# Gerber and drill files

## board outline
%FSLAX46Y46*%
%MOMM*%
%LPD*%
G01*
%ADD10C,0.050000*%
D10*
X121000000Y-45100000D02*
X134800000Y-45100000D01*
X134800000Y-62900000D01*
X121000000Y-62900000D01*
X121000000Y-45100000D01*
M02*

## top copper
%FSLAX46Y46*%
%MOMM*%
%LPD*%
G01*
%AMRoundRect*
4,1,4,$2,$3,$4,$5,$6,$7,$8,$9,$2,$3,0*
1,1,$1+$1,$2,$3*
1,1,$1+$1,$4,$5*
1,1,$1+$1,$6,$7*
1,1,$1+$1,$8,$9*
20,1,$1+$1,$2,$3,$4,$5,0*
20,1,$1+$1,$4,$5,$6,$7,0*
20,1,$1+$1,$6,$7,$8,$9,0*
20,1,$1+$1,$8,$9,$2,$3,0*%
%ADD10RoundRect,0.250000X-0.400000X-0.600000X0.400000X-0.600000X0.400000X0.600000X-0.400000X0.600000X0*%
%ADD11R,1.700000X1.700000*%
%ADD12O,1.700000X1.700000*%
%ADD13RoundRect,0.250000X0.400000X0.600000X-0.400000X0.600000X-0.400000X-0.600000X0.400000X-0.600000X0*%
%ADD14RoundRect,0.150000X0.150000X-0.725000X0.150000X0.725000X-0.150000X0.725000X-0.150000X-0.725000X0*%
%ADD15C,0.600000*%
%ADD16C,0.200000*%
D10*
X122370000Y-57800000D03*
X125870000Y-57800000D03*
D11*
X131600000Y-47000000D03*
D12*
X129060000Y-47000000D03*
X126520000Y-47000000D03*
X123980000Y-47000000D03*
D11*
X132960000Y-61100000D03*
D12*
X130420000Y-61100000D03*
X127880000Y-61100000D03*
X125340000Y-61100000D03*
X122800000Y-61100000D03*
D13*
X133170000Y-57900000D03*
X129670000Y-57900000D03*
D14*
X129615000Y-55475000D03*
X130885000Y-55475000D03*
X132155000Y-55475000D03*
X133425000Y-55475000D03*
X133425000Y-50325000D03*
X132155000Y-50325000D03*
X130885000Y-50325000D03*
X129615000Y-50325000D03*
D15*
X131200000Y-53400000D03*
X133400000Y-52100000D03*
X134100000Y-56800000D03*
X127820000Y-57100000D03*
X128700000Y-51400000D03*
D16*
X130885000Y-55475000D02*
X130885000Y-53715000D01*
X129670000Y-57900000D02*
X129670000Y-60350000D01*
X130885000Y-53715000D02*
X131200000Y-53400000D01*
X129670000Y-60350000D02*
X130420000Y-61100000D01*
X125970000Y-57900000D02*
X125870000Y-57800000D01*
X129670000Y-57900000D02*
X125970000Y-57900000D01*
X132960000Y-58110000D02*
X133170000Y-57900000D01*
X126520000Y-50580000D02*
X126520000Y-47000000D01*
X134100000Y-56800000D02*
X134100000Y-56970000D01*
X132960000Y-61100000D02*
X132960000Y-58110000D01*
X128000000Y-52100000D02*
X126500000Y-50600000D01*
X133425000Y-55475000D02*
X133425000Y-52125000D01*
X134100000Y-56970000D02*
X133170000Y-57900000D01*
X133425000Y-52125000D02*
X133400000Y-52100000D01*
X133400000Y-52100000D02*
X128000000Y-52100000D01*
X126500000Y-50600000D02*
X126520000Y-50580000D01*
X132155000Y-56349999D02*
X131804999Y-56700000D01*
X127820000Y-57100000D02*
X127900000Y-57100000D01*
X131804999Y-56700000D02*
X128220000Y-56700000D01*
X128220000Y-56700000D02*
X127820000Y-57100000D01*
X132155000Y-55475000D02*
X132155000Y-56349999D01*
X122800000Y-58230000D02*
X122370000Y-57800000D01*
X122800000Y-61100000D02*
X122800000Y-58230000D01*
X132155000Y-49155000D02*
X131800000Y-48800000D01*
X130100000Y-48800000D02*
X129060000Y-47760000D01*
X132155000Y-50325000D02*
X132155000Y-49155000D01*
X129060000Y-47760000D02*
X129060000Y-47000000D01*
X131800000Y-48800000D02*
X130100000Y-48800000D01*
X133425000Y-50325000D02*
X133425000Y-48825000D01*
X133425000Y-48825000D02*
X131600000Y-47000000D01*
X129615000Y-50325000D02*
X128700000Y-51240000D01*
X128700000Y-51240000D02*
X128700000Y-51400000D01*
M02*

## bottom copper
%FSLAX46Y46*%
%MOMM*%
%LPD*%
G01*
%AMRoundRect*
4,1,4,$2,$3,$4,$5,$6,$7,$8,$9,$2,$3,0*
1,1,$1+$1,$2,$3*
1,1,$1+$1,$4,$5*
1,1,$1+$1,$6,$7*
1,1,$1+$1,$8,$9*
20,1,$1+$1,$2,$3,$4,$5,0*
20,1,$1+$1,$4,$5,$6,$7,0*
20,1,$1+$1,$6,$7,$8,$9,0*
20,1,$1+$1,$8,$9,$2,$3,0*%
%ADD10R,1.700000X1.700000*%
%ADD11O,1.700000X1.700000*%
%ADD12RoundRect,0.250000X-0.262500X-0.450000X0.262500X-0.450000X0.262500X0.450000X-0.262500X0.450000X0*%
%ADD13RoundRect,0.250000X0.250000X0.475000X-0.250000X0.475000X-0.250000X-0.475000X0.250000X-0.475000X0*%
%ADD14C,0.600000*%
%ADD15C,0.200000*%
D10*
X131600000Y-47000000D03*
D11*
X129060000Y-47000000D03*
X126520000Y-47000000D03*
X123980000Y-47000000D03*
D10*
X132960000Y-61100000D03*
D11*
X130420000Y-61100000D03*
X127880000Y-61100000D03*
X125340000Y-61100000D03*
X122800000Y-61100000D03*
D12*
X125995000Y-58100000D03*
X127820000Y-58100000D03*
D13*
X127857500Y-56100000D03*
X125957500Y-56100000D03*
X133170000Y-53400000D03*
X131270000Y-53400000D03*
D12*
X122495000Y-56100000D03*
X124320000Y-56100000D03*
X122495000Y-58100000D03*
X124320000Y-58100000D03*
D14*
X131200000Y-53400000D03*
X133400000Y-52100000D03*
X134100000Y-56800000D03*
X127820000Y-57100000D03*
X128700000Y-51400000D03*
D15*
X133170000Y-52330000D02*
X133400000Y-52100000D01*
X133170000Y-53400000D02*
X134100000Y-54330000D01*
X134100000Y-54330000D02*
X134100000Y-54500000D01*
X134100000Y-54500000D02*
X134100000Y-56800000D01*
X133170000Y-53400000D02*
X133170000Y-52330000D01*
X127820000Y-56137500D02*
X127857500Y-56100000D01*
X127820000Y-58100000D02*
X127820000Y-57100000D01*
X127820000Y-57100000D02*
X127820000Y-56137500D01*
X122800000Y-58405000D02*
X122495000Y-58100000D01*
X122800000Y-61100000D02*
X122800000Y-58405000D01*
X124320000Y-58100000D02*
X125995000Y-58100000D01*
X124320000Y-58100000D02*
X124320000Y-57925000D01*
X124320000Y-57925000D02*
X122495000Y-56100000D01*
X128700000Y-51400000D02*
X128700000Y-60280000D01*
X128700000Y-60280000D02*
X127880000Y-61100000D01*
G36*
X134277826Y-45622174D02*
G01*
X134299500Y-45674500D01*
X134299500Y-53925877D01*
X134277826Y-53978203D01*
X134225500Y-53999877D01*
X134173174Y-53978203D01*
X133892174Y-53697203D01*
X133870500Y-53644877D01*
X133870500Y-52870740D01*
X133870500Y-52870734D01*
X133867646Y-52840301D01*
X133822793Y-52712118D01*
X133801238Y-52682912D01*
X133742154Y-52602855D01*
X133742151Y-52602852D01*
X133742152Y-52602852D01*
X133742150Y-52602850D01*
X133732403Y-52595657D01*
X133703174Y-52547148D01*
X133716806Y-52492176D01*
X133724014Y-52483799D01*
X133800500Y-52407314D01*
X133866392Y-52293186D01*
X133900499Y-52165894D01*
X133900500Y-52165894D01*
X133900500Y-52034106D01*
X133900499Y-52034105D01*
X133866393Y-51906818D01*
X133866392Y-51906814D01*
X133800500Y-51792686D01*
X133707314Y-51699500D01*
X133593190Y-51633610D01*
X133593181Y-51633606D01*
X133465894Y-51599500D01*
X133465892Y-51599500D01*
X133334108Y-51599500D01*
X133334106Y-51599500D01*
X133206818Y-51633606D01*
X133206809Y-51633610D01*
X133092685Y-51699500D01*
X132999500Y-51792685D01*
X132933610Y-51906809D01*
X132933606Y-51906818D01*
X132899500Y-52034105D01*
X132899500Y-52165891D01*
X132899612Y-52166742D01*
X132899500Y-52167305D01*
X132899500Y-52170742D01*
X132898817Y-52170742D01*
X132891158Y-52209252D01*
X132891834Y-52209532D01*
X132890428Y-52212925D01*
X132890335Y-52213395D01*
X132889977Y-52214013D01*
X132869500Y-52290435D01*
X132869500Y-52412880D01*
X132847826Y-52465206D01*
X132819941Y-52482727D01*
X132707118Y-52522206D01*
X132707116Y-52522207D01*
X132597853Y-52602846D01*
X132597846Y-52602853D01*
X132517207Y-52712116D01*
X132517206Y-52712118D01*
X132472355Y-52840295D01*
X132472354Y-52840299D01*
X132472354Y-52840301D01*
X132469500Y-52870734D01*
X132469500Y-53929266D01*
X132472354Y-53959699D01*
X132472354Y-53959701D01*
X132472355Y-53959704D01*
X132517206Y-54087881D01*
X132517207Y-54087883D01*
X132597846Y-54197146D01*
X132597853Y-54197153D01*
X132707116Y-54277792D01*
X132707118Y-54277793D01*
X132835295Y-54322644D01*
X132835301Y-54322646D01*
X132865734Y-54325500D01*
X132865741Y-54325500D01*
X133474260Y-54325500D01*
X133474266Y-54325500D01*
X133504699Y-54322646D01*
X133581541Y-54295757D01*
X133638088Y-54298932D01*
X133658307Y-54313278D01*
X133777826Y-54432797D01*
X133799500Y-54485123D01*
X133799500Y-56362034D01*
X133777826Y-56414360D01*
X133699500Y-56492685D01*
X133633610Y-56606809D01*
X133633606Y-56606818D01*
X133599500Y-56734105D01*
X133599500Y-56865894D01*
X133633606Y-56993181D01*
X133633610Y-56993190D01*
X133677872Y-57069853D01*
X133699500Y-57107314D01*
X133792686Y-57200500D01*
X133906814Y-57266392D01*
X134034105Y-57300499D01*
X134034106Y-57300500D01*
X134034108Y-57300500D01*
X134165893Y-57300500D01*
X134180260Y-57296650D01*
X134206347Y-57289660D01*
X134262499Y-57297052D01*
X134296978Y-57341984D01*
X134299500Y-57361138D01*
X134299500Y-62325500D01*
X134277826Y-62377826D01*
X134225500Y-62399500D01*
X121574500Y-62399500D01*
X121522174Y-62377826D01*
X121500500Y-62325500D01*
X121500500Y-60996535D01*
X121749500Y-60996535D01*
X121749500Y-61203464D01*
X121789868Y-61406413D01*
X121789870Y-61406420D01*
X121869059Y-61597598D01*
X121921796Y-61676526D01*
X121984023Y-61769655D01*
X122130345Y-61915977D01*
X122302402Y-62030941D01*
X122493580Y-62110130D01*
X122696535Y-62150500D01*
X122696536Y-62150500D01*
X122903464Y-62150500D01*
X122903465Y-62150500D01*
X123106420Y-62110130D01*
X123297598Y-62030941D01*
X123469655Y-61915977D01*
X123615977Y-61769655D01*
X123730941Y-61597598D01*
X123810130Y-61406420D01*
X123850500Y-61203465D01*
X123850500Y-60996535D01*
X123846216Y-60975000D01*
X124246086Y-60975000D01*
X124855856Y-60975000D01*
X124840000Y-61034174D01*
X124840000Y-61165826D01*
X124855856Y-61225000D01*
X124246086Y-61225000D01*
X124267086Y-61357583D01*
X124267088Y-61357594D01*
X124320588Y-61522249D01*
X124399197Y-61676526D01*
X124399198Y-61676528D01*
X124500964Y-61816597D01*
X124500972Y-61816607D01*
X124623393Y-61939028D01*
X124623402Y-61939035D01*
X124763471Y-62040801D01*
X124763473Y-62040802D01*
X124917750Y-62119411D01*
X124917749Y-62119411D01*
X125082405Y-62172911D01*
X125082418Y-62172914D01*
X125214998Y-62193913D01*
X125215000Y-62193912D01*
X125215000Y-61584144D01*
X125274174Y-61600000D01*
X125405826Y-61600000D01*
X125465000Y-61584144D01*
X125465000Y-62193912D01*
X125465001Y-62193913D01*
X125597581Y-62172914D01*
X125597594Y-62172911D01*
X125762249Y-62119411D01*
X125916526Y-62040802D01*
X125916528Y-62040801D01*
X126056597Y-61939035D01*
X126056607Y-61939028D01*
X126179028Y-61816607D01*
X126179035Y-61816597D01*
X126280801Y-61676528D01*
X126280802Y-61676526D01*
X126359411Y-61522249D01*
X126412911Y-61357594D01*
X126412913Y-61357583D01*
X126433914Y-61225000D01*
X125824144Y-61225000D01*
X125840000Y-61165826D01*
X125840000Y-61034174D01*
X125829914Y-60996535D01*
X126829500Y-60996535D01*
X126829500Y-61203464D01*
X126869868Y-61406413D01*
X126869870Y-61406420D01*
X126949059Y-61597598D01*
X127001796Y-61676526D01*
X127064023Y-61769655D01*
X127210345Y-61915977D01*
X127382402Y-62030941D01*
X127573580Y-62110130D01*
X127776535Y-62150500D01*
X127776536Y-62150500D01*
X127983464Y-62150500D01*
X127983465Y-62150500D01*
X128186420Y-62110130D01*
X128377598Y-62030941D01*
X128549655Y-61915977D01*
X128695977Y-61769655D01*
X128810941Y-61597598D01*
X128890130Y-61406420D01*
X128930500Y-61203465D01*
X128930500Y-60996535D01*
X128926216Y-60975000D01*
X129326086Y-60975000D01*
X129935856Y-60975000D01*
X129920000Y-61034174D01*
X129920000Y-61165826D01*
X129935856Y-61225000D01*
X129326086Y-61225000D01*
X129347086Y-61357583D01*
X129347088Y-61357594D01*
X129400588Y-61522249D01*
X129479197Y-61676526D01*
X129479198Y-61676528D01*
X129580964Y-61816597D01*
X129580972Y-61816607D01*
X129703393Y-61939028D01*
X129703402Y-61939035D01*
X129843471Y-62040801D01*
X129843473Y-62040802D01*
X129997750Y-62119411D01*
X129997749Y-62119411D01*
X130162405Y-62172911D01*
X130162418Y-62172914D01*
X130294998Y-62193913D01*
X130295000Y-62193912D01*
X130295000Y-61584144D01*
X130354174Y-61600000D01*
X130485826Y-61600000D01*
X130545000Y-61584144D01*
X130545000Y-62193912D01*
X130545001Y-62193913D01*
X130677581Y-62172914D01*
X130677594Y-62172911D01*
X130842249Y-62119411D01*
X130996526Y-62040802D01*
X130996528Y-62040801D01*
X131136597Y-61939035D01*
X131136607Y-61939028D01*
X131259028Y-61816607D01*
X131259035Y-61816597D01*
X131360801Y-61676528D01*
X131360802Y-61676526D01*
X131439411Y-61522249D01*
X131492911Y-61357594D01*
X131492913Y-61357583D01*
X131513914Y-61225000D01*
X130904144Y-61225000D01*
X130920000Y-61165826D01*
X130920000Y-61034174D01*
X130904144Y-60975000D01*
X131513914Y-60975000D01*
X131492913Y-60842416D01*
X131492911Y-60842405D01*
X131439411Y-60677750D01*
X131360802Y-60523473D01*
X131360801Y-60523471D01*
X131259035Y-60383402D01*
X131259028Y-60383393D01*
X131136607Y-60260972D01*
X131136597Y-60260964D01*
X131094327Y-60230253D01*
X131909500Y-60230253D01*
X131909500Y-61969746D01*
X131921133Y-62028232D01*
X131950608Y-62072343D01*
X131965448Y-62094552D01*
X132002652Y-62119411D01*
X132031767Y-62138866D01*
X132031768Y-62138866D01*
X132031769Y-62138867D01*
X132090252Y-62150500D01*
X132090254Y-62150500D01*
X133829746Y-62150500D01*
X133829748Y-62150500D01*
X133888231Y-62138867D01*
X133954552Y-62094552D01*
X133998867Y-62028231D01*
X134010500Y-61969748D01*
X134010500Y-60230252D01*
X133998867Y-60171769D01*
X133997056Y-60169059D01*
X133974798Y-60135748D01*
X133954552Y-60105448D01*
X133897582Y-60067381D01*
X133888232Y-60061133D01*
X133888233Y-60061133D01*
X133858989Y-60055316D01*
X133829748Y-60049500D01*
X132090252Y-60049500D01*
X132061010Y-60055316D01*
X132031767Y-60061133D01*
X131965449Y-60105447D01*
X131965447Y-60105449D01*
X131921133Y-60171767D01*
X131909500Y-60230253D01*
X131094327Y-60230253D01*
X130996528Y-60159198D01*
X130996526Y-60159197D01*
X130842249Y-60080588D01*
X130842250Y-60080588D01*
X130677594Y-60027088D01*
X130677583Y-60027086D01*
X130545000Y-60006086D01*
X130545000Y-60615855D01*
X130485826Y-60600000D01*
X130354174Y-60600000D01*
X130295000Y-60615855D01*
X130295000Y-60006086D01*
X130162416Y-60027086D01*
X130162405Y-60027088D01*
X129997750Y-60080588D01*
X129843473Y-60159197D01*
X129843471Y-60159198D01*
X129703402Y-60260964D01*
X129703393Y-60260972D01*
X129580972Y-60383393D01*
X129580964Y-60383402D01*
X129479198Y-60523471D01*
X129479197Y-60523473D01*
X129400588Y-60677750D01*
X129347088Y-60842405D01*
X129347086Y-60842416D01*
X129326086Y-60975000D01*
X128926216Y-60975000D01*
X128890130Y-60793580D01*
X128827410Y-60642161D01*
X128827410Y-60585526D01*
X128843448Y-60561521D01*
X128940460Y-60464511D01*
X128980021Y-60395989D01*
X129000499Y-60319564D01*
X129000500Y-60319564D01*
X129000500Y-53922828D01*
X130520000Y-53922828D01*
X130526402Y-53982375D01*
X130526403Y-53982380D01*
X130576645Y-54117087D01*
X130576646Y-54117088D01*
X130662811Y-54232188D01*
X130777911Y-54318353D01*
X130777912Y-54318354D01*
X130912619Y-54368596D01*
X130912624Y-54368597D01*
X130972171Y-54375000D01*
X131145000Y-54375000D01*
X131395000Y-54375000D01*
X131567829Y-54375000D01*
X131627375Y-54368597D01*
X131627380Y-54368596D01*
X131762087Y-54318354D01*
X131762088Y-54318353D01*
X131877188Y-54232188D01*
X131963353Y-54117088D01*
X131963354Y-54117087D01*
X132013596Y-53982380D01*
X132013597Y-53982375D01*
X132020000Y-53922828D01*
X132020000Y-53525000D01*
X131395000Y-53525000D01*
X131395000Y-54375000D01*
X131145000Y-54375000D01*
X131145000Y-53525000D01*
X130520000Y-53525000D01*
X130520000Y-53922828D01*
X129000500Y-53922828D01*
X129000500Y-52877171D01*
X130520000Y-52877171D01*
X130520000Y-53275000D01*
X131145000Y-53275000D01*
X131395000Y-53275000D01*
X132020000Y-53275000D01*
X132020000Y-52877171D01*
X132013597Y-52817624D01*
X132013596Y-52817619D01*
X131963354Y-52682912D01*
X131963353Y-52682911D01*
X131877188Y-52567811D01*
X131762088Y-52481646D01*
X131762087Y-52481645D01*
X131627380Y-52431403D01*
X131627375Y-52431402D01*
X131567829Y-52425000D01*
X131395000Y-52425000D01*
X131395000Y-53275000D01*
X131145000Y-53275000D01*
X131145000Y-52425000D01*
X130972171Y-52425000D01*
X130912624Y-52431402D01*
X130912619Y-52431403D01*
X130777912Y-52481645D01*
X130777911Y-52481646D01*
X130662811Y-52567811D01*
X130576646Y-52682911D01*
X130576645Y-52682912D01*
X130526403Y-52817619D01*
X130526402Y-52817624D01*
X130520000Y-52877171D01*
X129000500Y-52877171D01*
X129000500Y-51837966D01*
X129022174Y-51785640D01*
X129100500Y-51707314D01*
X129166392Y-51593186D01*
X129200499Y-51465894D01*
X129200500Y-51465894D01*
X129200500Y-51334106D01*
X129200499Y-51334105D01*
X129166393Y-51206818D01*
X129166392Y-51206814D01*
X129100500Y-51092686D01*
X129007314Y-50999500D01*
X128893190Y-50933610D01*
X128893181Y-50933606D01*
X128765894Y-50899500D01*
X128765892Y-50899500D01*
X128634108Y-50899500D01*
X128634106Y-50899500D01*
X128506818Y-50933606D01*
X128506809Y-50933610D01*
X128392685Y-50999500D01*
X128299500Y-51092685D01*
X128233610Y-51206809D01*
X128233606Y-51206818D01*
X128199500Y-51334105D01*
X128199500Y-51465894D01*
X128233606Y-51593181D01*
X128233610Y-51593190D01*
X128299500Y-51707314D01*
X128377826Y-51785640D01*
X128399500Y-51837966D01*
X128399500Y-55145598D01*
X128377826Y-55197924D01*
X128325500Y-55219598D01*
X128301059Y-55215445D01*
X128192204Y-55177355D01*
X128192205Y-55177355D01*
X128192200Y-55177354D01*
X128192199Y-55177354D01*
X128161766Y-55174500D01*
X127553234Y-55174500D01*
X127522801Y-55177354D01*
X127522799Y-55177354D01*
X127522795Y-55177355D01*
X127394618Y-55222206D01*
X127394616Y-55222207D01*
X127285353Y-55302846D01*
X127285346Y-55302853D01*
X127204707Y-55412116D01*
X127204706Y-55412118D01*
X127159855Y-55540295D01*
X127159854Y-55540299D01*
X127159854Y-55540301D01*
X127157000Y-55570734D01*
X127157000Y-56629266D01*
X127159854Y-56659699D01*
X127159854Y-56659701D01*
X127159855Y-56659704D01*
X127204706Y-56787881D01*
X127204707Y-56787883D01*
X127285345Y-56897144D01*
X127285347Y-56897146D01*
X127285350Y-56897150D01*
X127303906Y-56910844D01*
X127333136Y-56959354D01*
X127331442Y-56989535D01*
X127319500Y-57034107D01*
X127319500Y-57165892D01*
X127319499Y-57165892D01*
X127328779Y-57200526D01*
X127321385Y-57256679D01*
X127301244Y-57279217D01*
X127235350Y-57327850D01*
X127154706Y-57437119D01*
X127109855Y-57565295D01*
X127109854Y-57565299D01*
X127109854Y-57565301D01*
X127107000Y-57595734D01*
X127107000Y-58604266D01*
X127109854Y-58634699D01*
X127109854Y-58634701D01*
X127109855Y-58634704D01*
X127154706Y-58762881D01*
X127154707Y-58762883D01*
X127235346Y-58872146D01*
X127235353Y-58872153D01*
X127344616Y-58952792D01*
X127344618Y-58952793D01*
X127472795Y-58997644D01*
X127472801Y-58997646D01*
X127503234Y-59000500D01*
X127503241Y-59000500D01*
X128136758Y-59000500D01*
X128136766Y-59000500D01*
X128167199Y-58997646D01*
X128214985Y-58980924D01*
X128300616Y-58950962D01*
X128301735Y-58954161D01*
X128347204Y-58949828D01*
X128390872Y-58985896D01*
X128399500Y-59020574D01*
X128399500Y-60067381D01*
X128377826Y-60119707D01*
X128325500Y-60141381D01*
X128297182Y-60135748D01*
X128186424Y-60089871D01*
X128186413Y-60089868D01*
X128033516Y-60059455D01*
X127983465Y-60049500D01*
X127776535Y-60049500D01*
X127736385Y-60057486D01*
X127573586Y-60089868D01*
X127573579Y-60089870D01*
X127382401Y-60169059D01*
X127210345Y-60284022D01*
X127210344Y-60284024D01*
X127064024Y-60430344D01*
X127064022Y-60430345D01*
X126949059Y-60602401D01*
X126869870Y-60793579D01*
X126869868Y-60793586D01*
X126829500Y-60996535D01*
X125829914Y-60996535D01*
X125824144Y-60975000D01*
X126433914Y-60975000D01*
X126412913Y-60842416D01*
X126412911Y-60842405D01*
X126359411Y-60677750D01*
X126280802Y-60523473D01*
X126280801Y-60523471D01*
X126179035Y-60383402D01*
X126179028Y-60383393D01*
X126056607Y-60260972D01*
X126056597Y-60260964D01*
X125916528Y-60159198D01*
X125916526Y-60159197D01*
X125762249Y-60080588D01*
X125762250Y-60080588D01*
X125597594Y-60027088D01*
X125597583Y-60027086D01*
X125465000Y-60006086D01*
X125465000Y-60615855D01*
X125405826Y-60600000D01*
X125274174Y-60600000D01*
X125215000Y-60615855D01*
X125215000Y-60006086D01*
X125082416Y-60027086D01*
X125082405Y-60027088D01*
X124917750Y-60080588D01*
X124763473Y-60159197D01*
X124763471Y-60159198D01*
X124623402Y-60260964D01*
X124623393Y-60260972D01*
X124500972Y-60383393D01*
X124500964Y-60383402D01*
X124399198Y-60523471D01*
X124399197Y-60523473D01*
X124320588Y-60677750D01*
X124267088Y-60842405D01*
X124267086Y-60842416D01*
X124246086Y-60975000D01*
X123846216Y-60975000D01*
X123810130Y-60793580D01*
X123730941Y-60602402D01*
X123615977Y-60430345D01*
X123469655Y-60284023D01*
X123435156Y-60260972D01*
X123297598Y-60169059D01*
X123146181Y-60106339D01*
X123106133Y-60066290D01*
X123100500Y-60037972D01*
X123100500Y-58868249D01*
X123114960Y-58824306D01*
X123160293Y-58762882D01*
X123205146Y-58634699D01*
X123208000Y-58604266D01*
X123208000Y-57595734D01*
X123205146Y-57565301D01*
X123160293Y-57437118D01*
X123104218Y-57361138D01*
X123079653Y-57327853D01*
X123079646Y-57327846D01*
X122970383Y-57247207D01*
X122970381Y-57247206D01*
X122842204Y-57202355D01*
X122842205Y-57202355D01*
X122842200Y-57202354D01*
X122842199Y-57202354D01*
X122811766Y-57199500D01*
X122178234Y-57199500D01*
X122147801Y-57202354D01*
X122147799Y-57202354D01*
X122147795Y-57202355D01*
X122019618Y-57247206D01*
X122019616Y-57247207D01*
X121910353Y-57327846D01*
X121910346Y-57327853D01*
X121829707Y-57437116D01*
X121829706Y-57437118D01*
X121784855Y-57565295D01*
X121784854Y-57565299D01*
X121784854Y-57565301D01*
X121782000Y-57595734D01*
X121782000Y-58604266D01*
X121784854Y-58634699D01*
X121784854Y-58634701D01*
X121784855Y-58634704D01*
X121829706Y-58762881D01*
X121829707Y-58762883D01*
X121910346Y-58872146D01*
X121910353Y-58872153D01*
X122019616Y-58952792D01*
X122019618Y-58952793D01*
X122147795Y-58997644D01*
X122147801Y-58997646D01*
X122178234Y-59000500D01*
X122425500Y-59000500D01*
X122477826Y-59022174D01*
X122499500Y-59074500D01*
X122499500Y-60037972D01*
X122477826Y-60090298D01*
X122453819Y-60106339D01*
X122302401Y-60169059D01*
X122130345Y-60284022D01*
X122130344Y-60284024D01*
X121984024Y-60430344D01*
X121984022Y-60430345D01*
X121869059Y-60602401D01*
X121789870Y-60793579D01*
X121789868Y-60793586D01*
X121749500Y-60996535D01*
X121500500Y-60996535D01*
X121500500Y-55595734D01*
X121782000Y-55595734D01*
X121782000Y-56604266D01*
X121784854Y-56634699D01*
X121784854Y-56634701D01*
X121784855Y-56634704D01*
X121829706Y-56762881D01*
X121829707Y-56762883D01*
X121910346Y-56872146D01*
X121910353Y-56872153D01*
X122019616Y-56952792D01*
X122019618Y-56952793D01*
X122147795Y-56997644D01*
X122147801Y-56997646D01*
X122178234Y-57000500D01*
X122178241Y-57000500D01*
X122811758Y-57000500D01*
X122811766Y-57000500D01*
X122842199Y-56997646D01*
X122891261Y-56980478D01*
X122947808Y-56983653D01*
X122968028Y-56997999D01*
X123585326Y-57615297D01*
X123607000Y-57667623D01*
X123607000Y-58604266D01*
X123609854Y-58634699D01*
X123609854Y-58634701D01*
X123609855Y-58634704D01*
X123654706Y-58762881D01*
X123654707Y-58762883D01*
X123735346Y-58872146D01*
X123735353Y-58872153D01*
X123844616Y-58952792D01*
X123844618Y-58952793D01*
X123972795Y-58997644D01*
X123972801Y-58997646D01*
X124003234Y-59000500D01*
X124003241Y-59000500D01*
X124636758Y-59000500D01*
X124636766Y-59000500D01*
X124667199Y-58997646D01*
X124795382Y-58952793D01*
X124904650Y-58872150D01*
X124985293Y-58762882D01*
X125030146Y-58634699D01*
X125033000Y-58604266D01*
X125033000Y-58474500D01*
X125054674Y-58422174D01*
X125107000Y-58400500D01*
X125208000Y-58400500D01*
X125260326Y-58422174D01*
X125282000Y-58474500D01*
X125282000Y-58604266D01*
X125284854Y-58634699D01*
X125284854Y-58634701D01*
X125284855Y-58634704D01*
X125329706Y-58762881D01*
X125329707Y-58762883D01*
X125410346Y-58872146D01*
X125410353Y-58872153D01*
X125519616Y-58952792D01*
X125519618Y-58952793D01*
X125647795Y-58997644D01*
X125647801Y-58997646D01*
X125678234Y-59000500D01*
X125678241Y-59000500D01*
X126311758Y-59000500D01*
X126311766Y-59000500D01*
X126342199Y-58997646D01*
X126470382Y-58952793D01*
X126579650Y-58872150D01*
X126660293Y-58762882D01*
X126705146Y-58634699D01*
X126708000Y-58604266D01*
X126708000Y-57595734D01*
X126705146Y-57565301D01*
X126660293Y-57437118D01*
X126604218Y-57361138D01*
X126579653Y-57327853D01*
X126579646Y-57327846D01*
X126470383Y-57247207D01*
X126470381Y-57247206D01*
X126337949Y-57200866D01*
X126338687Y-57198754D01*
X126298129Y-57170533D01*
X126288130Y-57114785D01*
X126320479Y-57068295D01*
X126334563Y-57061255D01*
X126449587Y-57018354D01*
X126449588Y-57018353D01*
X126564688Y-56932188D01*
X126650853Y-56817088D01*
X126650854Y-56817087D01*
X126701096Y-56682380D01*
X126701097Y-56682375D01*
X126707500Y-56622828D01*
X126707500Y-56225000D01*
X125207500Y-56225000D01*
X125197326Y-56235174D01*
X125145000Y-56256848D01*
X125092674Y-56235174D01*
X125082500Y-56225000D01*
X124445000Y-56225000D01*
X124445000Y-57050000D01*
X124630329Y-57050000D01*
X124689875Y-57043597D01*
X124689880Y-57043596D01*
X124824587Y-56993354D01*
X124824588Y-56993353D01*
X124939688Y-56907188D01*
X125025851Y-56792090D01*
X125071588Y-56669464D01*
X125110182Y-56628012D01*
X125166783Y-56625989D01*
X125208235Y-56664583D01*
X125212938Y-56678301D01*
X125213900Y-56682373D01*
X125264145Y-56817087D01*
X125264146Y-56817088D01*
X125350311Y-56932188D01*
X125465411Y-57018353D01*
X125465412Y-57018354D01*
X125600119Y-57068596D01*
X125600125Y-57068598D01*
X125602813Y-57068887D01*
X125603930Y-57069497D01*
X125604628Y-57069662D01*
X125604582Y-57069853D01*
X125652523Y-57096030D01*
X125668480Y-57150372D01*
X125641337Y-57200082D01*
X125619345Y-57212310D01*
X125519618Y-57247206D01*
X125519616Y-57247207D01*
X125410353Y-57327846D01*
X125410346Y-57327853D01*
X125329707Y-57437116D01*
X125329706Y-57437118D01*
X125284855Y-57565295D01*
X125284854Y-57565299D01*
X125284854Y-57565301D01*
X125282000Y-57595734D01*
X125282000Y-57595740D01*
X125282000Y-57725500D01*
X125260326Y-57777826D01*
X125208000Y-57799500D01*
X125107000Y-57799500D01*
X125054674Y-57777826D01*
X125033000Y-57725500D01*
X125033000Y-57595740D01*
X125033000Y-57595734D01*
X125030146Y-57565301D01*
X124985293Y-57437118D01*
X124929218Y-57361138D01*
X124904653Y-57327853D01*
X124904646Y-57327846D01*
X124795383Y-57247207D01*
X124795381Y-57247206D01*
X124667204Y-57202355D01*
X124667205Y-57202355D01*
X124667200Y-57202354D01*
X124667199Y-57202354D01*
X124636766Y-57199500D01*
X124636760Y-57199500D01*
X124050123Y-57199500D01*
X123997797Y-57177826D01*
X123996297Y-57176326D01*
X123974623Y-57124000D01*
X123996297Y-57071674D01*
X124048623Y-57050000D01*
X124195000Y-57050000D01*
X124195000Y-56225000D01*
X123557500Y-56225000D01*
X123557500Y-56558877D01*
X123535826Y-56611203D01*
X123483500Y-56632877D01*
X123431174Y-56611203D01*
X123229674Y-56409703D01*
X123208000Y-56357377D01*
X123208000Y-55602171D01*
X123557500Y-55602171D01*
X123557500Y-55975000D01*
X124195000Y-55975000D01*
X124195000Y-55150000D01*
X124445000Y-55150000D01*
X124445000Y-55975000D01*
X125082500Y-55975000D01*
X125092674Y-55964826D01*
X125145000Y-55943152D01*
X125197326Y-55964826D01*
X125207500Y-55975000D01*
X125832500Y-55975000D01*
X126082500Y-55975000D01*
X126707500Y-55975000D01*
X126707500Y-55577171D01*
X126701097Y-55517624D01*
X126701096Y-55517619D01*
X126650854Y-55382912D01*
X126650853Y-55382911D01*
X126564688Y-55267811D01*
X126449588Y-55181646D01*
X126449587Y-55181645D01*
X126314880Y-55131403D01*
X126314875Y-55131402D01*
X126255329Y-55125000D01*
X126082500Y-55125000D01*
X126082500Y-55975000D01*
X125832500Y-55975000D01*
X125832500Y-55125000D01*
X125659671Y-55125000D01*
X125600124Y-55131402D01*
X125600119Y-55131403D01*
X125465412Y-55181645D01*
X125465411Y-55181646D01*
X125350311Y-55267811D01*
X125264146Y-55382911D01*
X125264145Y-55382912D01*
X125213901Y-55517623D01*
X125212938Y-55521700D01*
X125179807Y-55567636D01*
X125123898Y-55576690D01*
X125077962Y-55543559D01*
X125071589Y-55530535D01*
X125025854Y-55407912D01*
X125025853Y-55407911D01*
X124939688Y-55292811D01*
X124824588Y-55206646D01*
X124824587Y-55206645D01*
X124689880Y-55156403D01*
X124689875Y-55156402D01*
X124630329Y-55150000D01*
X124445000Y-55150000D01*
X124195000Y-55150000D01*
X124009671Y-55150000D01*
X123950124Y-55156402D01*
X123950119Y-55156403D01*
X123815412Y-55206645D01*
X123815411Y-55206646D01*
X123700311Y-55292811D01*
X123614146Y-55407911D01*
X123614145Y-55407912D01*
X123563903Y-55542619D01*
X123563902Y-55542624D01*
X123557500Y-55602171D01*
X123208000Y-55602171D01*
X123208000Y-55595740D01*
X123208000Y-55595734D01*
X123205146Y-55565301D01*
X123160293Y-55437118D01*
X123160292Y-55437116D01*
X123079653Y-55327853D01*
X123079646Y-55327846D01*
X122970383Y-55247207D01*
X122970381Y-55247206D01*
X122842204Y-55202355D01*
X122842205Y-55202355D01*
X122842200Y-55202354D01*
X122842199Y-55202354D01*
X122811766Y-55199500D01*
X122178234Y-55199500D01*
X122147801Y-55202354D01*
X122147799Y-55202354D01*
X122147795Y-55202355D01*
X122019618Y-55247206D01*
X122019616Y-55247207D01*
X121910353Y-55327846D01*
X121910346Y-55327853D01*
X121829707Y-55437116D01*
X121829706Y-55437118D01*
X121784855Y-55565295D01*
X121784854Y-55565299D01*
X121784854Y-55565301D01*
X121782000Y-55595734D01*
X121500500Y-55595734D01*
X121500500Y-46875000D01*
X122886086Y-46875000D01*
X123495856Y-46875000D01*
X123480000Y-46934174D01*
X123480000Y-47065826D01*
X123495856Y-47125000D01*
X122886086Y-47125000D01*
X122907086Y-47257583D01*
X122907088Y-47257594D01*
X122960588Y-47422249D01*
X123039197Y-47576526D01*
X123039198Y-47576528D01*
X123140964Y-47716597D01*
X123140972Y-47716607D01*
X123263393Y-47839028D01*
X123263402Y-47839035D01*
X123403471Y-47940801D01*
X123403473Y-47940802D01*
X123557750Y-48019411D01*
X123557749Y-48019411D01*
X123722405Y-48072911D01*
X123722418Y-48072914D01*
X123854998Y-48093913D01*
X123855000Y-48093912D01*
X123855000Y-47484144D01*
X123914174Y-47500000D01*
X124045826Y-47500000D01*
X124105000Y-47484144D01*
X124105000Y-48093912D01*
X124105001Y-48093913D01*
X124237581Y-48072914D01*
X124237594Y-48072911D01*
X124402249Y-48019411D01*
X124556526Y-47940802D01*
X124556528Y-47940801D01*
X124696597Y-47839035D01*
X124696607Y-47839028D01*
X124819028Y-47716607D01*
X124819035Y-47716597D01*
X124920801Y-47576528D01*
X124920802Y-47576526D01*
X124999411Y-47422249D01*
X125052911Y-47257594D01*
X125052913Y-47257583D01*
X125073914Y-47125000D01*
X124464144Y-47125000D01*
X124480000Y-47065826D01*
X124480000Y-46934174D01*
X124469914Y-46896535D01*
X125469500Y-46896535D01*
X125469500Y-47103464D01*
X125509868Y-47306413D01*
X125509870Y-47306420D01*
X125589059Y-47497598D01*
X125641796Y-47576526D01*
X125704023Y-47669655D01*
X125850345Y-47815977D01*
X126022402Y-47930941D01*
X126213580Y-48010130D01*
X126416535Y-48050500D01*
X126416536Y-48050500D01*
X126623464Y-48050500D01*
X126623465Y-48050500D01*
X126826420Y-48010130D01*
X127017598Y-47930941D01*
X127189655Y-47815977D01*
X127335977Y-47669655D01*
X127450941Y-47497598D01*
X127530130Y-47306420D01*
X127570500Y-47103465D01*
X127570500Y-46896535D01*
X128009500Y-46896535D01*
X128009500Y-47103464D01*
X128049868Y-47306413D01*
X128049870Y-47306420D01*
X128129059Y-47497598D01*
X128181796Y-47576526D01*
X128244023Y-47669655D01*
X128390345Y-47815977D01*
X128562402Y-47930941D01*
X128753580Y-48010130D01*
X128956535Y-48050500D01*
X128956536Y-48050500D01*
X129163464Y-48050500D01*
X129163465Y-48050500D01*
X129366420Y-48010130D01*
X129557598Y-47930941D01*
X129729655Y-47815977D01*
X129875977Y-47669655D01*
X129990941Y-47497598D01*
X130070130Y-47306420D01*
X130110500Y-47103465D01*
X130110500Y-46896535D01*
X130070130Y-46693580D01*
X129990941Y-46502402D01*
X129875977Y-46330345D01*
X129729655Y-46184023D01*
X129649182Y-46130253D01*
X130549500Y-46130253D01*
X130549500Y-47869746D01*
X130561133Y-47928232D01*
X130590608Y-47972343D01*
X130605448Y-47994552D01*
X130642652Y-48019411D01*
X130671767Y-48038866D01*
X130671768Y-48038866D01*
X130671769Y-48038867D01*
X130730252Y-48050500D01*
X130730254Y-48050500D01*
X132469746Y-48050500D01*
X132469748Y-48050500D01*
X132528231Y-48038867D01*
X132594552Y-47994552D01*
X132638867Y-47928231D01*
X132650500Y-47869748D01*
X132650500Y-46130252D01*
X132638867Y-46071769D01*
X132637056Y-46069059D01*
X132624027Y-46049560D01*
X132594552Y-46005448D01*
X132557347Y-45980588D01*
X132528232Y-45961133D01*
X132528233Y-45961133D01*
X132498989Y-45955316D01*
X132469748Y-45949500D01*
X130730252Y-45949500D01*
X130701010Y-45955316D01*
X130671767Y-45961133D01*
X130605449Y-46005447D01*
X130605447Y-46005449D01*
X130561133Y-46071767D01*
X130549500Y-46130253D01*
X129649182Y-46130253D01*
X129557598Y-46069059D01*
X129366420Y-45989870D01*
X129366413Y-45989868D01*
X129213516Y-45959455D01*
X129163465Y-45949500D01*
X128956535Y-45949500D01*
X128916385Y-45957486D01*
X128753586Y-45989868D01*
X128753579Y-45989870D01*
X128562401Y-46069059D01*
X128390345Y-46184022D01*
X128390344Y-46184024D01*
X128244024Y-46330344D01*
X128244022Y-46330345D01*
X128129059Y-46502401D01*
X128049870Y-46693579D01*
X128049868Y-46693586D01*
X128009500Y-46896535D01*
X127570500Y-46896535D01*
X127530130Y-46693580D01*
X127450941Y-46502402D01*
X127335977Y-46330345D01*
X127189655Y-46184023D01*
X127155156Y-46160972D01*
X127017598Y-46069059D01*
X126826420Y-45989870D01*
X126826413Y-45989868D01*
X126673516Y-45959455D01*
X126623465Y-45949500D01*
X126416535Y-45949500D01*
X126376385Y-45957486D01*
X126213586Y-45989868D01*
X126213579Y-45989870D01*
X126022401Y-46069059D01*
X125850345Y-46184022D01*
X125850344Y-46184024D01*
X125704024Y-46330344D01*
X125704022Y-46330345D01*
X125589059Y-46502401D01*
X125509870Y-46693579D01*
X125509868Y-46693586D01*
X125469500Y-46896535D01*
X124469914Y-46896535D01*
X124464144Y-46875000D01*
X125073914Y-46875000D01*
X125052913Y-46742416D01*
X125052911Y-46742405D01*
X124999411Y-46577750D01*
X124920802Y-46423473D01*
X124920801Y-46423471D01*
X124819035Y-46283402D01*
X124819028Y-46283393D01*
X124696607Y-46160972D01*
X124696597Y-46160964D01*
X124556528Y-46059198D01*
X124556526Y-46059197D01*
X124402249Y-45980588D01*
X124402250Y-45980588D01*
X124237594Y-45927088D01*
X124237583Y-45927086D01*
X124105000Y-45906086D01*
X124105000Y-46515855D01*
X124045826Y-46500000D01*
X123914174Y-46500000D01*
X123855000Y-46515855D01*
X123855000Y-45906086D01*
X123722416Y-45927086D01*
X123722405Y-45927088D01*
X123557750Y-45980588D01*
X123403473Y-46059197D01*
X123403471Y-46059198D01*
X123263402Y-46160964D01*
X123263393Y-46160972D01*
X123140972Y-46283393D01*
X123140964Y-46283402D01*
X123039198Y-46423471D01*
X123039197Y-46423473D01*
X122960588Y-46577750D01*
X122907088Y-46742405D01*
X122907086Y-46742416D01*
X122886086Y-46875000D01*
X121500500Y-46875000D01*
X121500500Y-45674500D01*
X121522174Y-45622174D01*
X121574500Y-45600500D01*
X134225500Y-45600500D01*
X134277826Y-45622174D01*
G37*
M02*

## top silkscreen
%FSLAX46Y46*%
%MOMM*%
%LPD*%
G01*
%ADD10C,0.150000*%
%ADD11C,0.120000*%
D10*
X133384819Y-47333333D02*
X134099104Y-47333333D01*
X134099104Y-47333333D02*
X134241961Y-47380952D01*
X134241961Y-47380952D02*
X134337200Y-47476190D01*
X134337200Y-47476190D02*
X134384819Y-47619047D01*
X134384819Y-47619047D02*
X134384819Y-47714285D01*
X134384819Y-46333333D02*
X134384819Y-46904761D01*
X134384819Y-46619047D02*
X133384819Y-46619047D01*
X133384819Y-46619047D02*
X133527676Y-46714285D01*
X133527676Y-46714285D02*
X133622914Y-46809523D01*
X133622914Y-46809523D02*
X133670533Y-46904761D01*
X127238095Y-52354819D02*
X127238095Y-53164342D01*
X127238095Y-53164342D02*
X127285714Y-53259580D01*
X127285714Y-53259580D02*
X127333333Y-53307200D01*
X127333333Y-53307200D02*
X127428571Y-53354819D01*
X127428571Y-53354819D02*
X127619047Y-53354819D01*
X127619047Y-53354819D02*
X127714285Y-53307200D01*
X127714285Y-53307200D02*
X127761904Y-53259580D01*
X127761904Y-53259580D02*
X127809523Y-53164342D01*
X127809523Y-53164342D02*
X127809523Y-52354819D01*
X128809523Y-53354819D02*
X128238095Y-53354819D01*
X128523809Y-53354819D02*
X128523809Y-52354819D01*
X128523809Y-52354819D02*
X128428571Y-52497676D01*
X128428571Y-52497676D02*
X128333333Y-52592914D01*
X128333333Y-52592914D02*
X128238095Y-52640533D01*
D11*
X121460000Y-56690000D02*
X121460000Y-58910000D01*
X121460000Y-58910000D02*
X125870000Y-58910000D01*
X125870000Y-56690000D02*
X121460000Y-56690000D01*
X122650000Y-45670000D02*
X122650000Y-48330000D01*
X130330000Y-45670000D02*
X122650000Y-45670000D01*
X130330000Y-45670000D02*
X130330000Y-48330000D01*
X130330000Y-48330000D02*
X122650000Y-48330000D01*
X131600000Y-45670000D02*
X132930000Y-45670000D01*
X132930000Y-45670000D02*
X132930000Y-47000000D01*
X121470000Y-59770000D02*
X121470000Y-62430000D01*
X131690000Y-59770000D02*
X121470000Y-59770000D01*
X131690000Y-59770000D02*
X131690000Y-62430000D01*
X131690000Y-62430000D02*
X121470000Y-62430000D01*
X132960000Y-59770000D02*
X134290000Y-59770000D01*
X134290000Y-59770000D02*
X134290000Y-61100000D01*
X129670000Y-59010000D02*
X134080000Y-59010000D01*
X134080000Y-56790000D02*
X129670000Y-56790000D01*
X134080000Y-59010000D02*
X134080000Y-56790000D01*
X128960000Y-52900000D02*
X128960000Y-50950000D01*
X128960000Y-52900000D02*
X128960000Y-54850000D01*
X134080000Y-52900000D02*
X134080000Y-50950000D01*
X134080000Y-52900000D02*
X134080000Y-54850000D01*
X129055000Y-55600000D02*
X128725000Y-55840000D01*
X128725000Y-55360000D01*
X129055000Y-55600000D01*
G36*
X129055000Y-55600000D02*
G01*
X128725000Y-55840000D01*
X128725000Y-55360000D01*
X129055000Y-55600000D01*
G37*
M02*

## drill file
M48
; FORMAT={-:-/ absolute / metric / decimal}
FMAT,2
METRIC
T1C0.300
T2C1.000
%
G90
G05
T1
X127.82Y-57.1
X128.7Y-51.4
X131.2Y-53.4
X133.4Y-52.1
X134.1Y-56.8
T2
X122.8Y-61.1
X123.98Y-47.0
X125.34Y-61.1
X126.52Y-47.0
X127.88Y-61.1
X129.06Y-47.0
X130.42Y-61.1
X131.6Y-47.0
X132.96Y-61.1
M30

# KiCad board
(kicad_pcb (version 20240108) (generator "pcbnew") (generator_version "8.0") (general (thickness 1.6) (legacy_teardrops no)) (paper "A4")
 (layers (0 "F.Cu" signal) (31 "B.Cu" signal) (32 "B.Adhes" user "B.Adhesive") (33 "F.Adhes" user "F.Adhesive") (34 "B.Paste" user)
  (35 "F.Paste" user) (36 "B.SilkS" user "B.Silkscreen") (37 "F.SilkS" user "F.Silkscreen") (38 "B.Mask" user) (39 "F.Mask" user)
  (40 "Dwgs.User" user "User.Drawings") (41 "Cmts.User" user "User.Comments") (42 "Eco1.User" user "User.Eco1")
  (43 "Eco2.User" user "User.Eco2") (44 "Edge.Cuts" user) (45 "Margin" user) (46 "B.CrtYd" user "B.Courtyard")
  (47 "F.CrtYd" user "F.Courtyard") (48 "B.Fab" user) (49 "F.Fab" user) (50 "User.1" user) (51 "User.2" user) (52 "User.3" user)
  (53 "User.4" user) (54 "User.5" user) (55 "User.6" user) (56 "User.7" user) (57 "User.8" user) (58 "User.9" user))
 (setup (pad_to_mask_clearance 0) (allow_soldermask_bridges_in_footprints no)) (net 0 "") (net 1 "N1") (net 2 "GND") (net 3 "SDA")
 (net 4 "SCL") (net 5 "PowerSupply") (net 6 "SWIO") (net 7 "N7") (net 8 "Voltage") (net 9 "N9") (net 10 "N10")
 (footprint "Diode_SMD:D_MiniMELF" (layer "F.Cu") (at 124.12 57.8)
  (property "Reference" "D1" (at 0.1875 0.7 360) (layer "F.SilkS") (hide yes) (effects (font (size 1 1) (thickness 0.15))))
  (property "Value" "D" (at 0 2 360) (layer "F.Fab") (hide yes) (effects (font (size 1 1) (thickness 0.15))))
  (fp_line (start -2.66 -1.11) (end -2.66 1.11) (stroke (width 0.12) (type solid)) (layer "F.SilkS"))
  (fp_line (start -2.66 1.11) (end 1.75 1.11) (stroke (width 0.12) (type solid)) (layer "F.SilkS"))
  (fp_line (start 1.75 -1.11) (end -2.66 -1.11) (stroke (width 0.12) (type solid)) (layer "F.SilkS"))
  (pad "1" smd roundrect (at -1.75 0) (size 1.3 1.7) (layers "F.Cu" "F.Paste" "F.Mask") (roundrect_rratio 0.1923076923) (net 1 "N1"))
  (pad "2" smd roundrect (at 1.75 0) (size 1.3 1.7) (layers "F.Cu" "F.Paste" "F.Mask") (roundrect_rratio 0.1923076923) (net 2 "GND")))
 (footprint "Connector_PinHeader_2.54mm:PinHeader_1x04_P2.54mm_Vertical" (layer "F.Cu") (at 131.6 47 -90)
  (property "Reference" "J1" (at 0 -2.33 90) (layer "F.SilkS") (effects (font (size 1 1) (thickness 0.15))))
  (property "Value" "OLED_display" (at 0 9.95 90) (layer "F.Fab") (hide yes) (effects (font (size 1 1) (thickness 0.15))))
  (fp_line (start -1.33 8.95) (end 1.33 8.95) (stroke (width 0.12) (type solid)) (layer "F.SilkS"))
  (fp_line (start -1.33 1.27) (end -1.33 8.95) (stroke (width 0.12) (type solid)) (layer "F.SilkS"))
  (fp_line (start -1.33 1.27) (end 1.33 1.27) (stroke (width 0.12) (type solid)) (layer "F.SilkS"))
  (fp_line (start 1.33 1.27) (end 1.33 8.95) (stroke (width 0.12) (type solid)) (layer "F.SilkS"))
  (fp_line (start -1.33 0) (end -1.33 -1.33) (stroke (width 0.12) (type solid)) (layer "F.SilkS"))
  (fp_line (start -1.33 -1.33) (end 0 -1.33) (stroke (width 0.12) (type solid)) (layer "F.SilkS"))
  (pad "1" thru_hole rect (at 0 0 270) (size 1.7 1.7) (drill 1) (layers "*.Cu" "*.Mask") (remove_unused_layers no) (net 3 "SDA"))
  (pad "2" thru_hole oval (at 0 2.54 270) (size 1.7 1.7) (drill 1) (layers "*.Cu" "*.Mask") (remove_unused_layers no) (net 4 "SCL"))
  (pad "3" thru_hole oval (at 0 5.08 270) (size 1.7 1.7) (drill 1) (layers "*.Cu" "*.Mask") (remove_unused_layers no) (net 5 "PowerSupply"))
  (pad "4" thru_hole oval (at 0 7.62 270) (size 1.7 1.7) (drill 1) (layers "*.Cu" "*.Mask") (remove_unused_layers no) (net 2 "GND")))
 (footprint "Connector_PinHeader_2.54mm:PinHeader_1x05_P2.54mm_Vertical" (layer "F.Cu") (at 132.96 61.1 -90)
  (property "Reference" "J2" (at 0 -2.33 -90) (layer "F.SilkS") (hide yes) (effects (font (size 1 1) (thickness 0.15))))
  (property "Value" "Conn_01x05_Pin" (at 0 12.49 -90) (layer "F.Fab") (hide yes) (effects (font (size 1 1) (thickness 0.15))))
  (fp_line (start -1.33 11.49) (end 1.33 11.49) (stroke (width 0.12) (type solid)) (layer "F.SilkS"))
  (fp_line (start -1.33 1.27) (end -1.33 11.49) (stroke (width 0.12) (type solid)) (layer "F.SilkS"))
  (fp_line (start -1.33 1.27) (end 1.33 1.27) (stroke (width 0.12) (type solid)) (layer "F.SilkS"))
  (fp_line (start 1.33 1.27) (end 1.33 11.49) (stroke (width 0.12) (type solid)) (layer "F.SilkS"))
  (fp_line (start -1.33 0) (end -1.33 -1.33) (stroke (width 0.12) (type solid)) (layer "F.SilkS"))
  (fp_line (start -1.33 -1.33) (end 0 -1.33) (stroke (width 0.12) (type solid)) (layer "F.SilkS"))
  (pad "1" thru_hole rect (at 0 0 270) (size 1.7 1.7) (drill 1) (layers "*.Cu" "*.Mask") (remove_unused_layers no) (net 5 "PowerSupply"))
  (pad "2" thru_hole oval (at 0 2.54 270) (size 1.7 1.7) (drill 1) (layers "*.Cu" "*.Mask") (remove_unused_layers no) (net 2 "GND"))
  (pad "3" thru_hole oval (at 0 5.08 270) (size 1.7 1.7) (drill 1) (layers "*.Cu" "*.Mask") (remove_unused_layers no) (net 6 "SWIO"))
  (pad "4" thru_hole oval (at 0 7.62 270) (size 1.7 1.7) (drill 1) (layers "*.Cu" "*.Mask") (remove_unused_layers no) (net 2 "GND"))
  (pad "5" thru_hole oval (at 0 10.16 270) (size 1.7 1.7) (drill 1) (layers "*.Cu" "*.Mask") (remove_unused_layers no) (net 1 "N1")))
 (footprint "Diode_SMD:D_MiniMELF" (layer "F.Cu") (at 131.42 57.9 180)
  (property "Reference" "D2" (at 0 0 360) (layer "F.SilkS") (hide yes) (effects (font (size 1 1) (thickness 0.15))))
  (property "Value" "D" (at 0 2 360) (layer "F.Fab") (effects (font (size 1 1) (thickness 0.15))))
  (fp_line (start 1.75 -1.11) (end -2.66 -1.11) (stroke (width 0.12) (type solid)) (layer "F.SilkS"))
  (fp_line (start -2.66 1.11) (end 1.75 1.11) (stroke (width 0.12) (type solid)) (layer "F.SilkS"))
  (fp_line (start -2.66 -1.11) (end -2.66 1.11) (stroke (width 0.12) (type solid)) (layer "F.SilkS"))
  (pad "1" smd roundrect (at -1.75 0 180) (size 1.3 1.7) (layers "F.Cu" "F.Paste" "F.Mask") (roundrect_rratio 0.1923076923)
   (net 5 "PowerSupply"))
  (pad "2" smd roundrect (at 1.75 0 180) (size 1.3 1.7) (layers "F.Cu" "F.Paste" "F.Mask") (roundrect_rratio 0.1923076923) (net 2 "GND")))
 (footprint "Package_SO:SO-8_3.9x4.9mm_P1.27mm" (layer "F.Cu") (at 131.52 52.9 90)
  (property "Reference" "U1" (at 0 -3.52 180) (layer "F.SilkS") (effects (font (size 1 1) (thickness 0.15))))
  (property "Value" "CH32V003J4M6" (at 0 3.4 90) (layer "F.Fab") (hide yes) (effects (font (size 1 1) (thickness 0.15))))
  (fp_line (start 0 -2.56) (end 1.95 -2.56) (stroke (width 0.12) (type solid)) (layer "F.SilkS"))
  (fp_line (start 0 -2.56) (end -1.95 -2.56) (stroke (width 0.12) (type solid)) (layer "F.SilkS"))
  (fp_line (start 0 2.56) (end 1.95 2.56) (stroke (width 0.12) (type solid)) (layer "F.SilkS"))
  (fp_line (start 0 2.56) (end -1.95 2.56) (stroke (width 0.12) (type solid)) (layer "F.SilkS"))
  (fp_poly
   (pts (xy -2.7 -2.465) (xy -2.94 -2.795) (xy -2.46 -2.795) (xy -2.7 -2.465)) (stroke (width 0.12) (type solid)) (fill solid)
   (layer "F.SilkS"))
  (pad "1" smd roundrect (at -2.575 -1.905 90) (size 1.75 0.6) (layers "F.Cu" "F.Paste" "F.Mask") (roundrect_rratio 0.25) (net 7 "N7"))
  (pad "2" smd roundrect (at -2.575 -0.635 90) (size 1.75 0.6) (layers "F.Cu" "F.Paste" "F.Mask") (roundrect_rratio 0.25) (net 2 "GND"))
  (pad "3" smd roundrect (at -2.575 0.635 90) (size 1.75 0.6) (layers "F.Cu" "F.Paste" "F.Mask") (roundrect_rratio 0.25) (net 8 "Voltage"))
  (pad "4" smd roundrect (at -2.575 1.905 90) (size 1.75 0.6) (layers "F.Cu" "F.Paste" "F.Mask") (roundrect_rratio 0.25)
   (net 5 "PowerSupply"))
  (pad "5" smd roundrect (at 2.575 1.905 90) (size 1.75 0.6) (layers "F.Cu" "F.Paste" "F.Mask") (roundrect_rratio 0.25) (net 3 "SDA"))
  (pad "6" smd roundrect (at 2.575 0.635 90) (size 1.75 0.6) (layers "F.Cu" "F.Paste" "F.Mask") (roundrect_rratio 0.25) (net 4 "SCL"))
  (pad "7" smd roundrect (at 2.575 -0.635 90) (size 1.75 0.6) (layers "F.Cu" "F.Paste" "F.Mask") (roundrect_rratio 0.25) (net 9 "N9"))
  (pad "8" smd roundrect (at 2.575 -1.905 90) (size 1.75 0.6) (layers "F.Cu" "F.Paste" "F.Mask") (roundrect_rratio 0.25) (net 6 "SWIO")))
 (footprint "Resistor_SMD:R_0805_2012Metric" (layer "B.Cu") (at 126.9075 58.1)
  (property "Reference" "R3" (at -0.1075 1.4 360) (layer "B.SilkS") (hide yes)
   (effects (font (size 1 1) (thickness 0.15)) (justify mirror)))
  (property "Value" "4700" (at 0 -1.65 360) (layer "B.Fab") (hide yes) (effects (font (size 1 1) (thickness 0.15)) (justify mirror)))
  (pad "1" smd roundrect (at -0.9125 0) (size 1.025 1.4) (layers "B.Cu" "B.Paste" "B.Mask") (roundrect_rratio 0.243902) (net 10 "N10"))
  (pad "2" smd roundrect (at 0.9125 0) (size 1.025 1.4) (layers "B.Cu" "B.Paste" "B.Mask") (roundrect_rratio 0.243902) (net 8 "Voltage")))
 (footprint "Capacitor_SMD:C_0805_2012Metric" (layer "B.Cu") (at 126.9075 56.1 180)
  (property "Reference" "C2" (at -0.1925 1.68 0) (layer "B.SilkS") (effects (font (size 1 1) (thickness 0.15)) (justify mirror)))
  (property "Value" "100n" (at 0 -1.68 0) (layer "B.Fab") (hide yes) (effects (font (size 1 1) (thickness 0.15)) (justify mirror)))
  (pad "1" smd roundrect (at -0.95 0 180) (size 1 1.45) (layers "B.Cu" "B.Paste" "B.Mask") (roundrect_rratio 0.25) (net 8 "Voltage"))
  (pad "2" smd roundrect (at 0.95 0 180) (size 1 1.45) (layers "B.Cu" "B.Paste" "B.Mask") (roundrect_rratio 0.25) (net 2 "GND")))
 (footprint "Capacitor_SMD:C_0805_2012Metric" (layer "B.Cu") (at 132.22 53.4 180)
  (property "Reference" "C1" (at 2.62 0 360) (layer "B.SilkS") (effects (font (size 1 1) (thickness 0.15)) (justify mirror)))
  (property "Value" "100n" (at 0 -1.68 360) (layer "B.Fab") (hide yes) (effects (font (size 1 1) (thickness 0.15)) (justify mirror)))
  (pad "1" smd roundrect (at -0.95 0 180) (size 1 1.45) (layers "B.Cu" "B.Paste" "B.Mask") (roundrect_rratio 0.25) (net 5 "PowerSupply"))
  (pad "2" smd roundrect (at 0.95 0 180) (size 1 1.45) (layers "B.Cu" "B.Paste" "B.Mask") (roundrect_rratio 0.25) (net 2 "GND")))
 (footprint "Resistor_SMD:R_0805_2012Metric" (layer "B.Cu") (at 123.4075 56.1)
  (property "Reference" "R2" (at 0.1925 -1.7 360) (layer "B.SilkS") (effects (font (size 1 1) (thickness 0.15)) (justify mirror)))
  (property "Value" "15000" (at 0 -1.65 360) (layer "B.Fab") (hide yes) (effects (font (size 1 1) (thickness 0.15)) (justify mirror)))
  (pad "1" smd roundrect (at -0.9125 0) (size 1.025 1.4) (layers "B.Cu" "B.Paste" "B.Mask") (roundrect_rratio 0.243902) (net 10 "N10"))
  (pad "2" smd roundrect (at 0.9125 0) (size 1.025 1.4) (layers "B.Cu" "B.Paste" "B.Mask") (roundrect_rratio 0.243902) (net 2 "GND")))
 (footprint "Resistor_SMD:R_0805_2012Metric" (layer "B.Cu") (at 123.4075 58.1)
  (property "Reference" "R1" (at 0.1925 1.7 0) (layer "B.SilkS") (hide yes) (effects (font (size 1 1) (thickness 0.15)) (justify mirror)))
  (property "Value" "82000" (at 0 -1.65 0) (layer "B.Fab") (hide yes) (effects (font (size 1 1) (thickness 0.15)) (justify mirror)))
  (pad "1" smd roundrect (at -0.9125 0) (size 1.025 1.4) (layers "B.Cu" "B.Paste" "B.Mask") (roundrect_rratio 0.243902) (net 1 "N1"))
  (pad "2" smd roundrect (at 0.9125 0) (size 1.025 1.4) (layers "B.Cu" "B.Paste" "B.Mask") (roundrect_rratio 0.243902) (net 10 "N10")))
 (gr_rect (start 121 45.1) (end 134.8 62.9) (stroke (width 0.05) (type default)) (fill none) (layer "Edge.Cuts"))
 (segment (start 130.885 55.475) (end 130.885 53.715) (width 0.2) (layer "F.Cu") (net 2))
 (segment (start 129.67 57.9) (end 129.67 60.35) (width 0.2) (layer "F.Cu") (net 2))
 (segment (start 130.885 53.715) (end 131.2 53.4) (width 0.2) (layer "F.Cu") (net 2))
 (segment (start 129.67 60.35) (end 130.42 61.1) (width 0.2) (layer "F.Cu") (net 2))
 (segment (start 125.97 57.9) (end 125.87 57.8) (width 0.2) (layer "F.Cu") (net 2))
 (segment (start 129.67 57.9) (end 125.97 57.9) (width 0.2) (layer "F.Cu") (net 2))
 (via (at 131.2 53.4) (size 0.6) (drill 0.3) (layers "F.Cu" "B.Cu") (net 2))
 (segment (start 132.96 58.11) (end 133.17 57.9) (width 0.2) (layer "F.Cu") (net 5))
 (segment (start 126.52 50.58) (end 126.52 47) (width 0.2) (layer "F.Cu") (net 5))
 (segment (start 134.1 56.8) (end 134.1 56.97) (width 0.2) (layer "F.Cu") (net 5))
 (segment (start 132.96 61.1) (end 132.96 58.11) (width 0.2) (layer "F.Cu") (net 5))
 (segment (start 128 52.1) (end 126.5 50.6) (width 0.2) (layer "F.Cu") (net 5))
 (segment (start 133.425 55.475) (end 133.425 52.125) (width 0.2) (layer "F.Cu") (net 5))
 (segment (start 134.1 56.97) (end 133.17 57.9) (width 0.2) (layer "F.Cu") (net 5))
 (segment (start 133.425 52.125) (end 133.4 52.1) (width 0.2) (layer "F.Cu") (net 5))
 (segment (start 133.4 52.1) (end 128 52.1) (width 0.2) (layer "F.Cu") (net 5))
 (segment (start 126.5 50.6) (end 126.52 50.58) (width 0.2) (layer "F.Cu") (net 5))
 (via (at 133.4 52.1) (size 0.6) (drill 0.3) (layers "F.Cu" "B.Cu") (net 5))
 (via (at 134.1 56.8) (size 0.6) (drill 0.3) (layers "F.Cu" "B.Cu") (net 5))
 (segment (start 133.17 52.33) (end 133.4 52.1) (width 0.2) (layer "B.Cu") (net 5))
 (segment (start 133.17 53.4) (end 134.1 54.33) (width 0.2) (layer "B.Cu") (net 5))
 (segment (start 134.1 54.33) (end 134.1 54.5) (width 0.2) (layer "B.Cu") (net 5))
 (segment (start 134.1 54.5) (end 134.1 56.8) (width 0.2) (layer "B.Cu") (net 5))
 (segment (start 133.17 53.4) (end 133.17 52.33) (width 0.2) (layer "B.Cu") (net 5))
 (segment (start 132.155 56.349999) (end 131.804999 56.7) (width 0.2) (layer "F.Cu") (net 8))
 (segment (start 127.82 57.1) (end 127.9 57.1) (width 0.2) (layer "F.Cu") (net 8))
 (segment (start 131.804999 56.7) (end 128.22 56.7) (width 0.2) (layer "F.Cu") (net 8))
 (segment (start 128.22 56.7) (end 127.82 57.1) (width 0.2) (layer "F.Cu") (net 8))
 (segment (start 132.155 55.475) (end 132.155 56.349999) (width 0.2) (layer "F.Cu") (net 8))
 (via (at 127.82 57.1) (size 0.6) (drill 0.3) (layers "F.Cu" "B.Cu") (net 8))
 (segment (start 127.82 56.1375) (end 127.8575 56.1) (width 0.2) (layer "B.Cu") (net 8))
 (segment (start 127.82 58.1) (end 127.82 57.1) (width 0.2) (layer "B.Cu") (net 8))
 (segment (start 127.82 57.1) (end 127.82 56.1375) (width 0.2) (layer "B.Cu") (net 8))
 (segment (start 122.8 58.23) (end 122.37 57.8) (width 0.2) (layer "F.Cu") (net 1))
 (segment (start 122.8 61.1) (end 122.8 58.23) (width 0.2) (layer "F.Cu") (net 1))
 (segment (start 122.8 58.405) (end 122.495 58.1) (width 0.2) (layer "B.Cu") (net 1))
 (segment (start 122.8 61.1) (end 122.8 58.405) (width 0.2) (layer "B.Cu") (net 1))
 (segment (start 132.155 49.155) (end 131.8 48.8) (width 0.2) (layer "F.Cu") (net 4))
 (segment (start 130.1 48.8) (end 129.06 47.76) (width 0.2) (layer "F.Cu") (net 4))
 (segment (start 132.155 50.325) (end 132.155 49.155) (width 0.2) (layer "F.Cu") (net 4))
 (segment (start 129.06 47.76) (end 129.06 47) (width 0.2) (layer "F.Cu") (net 4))
 (segment (start 131.8 48.8) (end 130.1 48.8) (width 0.2) (layer "F.Cu") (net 4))
 (segment (start 133.425 50.325) (end 133.425 48.825) (width 0.2) (layer "F.Cu") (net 3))
 (segment (start 133.425 48.825) (end 131.6 47) (width 0.2) (layer "F.Cu") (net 3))
 (segment (start 124.32 58.1) (end 125.995 58.1) (width 0.2) (layer "B.Cu") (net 10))
 (segment (start 124.32 58.1) (end 124.32 57.925) (width 0.2) (layer "B.Cu") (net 10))
 (segment (start 124.32 57.925) (end 122.495 56.1) (width 0.2) (layer "B.Cu") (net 10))
 (segment (start 129.615 50.325) (end 128.7 51.24) (width 0.2) (layer "F.Cu") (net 6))
 (segment (start 128.7 51.24) (end 128.7 51.4) (width 0.2) (layer "F.Cu") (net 6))
 (via (at 128.7 51.4) (size 0.6) (drill 0.3) (layers "F.Cu" "B.Cu") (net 6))
 (segment (start 128.7 51.4) (end 128.7 60.28) (width 0.2) (layer "B.Cu") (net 6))
 (segment (start 128.7 60.28) (end 127.88 61.1) (width 0.2) (layer "B.Cu") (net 6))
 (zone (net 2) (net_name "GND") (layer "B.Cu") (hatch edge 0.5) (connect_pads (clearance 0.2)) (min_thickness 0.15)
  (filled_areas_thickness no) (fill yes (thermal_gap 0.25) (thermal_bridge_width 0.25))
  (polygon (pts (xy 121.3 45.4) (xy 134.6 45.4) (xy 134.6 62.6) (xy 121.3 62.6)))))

